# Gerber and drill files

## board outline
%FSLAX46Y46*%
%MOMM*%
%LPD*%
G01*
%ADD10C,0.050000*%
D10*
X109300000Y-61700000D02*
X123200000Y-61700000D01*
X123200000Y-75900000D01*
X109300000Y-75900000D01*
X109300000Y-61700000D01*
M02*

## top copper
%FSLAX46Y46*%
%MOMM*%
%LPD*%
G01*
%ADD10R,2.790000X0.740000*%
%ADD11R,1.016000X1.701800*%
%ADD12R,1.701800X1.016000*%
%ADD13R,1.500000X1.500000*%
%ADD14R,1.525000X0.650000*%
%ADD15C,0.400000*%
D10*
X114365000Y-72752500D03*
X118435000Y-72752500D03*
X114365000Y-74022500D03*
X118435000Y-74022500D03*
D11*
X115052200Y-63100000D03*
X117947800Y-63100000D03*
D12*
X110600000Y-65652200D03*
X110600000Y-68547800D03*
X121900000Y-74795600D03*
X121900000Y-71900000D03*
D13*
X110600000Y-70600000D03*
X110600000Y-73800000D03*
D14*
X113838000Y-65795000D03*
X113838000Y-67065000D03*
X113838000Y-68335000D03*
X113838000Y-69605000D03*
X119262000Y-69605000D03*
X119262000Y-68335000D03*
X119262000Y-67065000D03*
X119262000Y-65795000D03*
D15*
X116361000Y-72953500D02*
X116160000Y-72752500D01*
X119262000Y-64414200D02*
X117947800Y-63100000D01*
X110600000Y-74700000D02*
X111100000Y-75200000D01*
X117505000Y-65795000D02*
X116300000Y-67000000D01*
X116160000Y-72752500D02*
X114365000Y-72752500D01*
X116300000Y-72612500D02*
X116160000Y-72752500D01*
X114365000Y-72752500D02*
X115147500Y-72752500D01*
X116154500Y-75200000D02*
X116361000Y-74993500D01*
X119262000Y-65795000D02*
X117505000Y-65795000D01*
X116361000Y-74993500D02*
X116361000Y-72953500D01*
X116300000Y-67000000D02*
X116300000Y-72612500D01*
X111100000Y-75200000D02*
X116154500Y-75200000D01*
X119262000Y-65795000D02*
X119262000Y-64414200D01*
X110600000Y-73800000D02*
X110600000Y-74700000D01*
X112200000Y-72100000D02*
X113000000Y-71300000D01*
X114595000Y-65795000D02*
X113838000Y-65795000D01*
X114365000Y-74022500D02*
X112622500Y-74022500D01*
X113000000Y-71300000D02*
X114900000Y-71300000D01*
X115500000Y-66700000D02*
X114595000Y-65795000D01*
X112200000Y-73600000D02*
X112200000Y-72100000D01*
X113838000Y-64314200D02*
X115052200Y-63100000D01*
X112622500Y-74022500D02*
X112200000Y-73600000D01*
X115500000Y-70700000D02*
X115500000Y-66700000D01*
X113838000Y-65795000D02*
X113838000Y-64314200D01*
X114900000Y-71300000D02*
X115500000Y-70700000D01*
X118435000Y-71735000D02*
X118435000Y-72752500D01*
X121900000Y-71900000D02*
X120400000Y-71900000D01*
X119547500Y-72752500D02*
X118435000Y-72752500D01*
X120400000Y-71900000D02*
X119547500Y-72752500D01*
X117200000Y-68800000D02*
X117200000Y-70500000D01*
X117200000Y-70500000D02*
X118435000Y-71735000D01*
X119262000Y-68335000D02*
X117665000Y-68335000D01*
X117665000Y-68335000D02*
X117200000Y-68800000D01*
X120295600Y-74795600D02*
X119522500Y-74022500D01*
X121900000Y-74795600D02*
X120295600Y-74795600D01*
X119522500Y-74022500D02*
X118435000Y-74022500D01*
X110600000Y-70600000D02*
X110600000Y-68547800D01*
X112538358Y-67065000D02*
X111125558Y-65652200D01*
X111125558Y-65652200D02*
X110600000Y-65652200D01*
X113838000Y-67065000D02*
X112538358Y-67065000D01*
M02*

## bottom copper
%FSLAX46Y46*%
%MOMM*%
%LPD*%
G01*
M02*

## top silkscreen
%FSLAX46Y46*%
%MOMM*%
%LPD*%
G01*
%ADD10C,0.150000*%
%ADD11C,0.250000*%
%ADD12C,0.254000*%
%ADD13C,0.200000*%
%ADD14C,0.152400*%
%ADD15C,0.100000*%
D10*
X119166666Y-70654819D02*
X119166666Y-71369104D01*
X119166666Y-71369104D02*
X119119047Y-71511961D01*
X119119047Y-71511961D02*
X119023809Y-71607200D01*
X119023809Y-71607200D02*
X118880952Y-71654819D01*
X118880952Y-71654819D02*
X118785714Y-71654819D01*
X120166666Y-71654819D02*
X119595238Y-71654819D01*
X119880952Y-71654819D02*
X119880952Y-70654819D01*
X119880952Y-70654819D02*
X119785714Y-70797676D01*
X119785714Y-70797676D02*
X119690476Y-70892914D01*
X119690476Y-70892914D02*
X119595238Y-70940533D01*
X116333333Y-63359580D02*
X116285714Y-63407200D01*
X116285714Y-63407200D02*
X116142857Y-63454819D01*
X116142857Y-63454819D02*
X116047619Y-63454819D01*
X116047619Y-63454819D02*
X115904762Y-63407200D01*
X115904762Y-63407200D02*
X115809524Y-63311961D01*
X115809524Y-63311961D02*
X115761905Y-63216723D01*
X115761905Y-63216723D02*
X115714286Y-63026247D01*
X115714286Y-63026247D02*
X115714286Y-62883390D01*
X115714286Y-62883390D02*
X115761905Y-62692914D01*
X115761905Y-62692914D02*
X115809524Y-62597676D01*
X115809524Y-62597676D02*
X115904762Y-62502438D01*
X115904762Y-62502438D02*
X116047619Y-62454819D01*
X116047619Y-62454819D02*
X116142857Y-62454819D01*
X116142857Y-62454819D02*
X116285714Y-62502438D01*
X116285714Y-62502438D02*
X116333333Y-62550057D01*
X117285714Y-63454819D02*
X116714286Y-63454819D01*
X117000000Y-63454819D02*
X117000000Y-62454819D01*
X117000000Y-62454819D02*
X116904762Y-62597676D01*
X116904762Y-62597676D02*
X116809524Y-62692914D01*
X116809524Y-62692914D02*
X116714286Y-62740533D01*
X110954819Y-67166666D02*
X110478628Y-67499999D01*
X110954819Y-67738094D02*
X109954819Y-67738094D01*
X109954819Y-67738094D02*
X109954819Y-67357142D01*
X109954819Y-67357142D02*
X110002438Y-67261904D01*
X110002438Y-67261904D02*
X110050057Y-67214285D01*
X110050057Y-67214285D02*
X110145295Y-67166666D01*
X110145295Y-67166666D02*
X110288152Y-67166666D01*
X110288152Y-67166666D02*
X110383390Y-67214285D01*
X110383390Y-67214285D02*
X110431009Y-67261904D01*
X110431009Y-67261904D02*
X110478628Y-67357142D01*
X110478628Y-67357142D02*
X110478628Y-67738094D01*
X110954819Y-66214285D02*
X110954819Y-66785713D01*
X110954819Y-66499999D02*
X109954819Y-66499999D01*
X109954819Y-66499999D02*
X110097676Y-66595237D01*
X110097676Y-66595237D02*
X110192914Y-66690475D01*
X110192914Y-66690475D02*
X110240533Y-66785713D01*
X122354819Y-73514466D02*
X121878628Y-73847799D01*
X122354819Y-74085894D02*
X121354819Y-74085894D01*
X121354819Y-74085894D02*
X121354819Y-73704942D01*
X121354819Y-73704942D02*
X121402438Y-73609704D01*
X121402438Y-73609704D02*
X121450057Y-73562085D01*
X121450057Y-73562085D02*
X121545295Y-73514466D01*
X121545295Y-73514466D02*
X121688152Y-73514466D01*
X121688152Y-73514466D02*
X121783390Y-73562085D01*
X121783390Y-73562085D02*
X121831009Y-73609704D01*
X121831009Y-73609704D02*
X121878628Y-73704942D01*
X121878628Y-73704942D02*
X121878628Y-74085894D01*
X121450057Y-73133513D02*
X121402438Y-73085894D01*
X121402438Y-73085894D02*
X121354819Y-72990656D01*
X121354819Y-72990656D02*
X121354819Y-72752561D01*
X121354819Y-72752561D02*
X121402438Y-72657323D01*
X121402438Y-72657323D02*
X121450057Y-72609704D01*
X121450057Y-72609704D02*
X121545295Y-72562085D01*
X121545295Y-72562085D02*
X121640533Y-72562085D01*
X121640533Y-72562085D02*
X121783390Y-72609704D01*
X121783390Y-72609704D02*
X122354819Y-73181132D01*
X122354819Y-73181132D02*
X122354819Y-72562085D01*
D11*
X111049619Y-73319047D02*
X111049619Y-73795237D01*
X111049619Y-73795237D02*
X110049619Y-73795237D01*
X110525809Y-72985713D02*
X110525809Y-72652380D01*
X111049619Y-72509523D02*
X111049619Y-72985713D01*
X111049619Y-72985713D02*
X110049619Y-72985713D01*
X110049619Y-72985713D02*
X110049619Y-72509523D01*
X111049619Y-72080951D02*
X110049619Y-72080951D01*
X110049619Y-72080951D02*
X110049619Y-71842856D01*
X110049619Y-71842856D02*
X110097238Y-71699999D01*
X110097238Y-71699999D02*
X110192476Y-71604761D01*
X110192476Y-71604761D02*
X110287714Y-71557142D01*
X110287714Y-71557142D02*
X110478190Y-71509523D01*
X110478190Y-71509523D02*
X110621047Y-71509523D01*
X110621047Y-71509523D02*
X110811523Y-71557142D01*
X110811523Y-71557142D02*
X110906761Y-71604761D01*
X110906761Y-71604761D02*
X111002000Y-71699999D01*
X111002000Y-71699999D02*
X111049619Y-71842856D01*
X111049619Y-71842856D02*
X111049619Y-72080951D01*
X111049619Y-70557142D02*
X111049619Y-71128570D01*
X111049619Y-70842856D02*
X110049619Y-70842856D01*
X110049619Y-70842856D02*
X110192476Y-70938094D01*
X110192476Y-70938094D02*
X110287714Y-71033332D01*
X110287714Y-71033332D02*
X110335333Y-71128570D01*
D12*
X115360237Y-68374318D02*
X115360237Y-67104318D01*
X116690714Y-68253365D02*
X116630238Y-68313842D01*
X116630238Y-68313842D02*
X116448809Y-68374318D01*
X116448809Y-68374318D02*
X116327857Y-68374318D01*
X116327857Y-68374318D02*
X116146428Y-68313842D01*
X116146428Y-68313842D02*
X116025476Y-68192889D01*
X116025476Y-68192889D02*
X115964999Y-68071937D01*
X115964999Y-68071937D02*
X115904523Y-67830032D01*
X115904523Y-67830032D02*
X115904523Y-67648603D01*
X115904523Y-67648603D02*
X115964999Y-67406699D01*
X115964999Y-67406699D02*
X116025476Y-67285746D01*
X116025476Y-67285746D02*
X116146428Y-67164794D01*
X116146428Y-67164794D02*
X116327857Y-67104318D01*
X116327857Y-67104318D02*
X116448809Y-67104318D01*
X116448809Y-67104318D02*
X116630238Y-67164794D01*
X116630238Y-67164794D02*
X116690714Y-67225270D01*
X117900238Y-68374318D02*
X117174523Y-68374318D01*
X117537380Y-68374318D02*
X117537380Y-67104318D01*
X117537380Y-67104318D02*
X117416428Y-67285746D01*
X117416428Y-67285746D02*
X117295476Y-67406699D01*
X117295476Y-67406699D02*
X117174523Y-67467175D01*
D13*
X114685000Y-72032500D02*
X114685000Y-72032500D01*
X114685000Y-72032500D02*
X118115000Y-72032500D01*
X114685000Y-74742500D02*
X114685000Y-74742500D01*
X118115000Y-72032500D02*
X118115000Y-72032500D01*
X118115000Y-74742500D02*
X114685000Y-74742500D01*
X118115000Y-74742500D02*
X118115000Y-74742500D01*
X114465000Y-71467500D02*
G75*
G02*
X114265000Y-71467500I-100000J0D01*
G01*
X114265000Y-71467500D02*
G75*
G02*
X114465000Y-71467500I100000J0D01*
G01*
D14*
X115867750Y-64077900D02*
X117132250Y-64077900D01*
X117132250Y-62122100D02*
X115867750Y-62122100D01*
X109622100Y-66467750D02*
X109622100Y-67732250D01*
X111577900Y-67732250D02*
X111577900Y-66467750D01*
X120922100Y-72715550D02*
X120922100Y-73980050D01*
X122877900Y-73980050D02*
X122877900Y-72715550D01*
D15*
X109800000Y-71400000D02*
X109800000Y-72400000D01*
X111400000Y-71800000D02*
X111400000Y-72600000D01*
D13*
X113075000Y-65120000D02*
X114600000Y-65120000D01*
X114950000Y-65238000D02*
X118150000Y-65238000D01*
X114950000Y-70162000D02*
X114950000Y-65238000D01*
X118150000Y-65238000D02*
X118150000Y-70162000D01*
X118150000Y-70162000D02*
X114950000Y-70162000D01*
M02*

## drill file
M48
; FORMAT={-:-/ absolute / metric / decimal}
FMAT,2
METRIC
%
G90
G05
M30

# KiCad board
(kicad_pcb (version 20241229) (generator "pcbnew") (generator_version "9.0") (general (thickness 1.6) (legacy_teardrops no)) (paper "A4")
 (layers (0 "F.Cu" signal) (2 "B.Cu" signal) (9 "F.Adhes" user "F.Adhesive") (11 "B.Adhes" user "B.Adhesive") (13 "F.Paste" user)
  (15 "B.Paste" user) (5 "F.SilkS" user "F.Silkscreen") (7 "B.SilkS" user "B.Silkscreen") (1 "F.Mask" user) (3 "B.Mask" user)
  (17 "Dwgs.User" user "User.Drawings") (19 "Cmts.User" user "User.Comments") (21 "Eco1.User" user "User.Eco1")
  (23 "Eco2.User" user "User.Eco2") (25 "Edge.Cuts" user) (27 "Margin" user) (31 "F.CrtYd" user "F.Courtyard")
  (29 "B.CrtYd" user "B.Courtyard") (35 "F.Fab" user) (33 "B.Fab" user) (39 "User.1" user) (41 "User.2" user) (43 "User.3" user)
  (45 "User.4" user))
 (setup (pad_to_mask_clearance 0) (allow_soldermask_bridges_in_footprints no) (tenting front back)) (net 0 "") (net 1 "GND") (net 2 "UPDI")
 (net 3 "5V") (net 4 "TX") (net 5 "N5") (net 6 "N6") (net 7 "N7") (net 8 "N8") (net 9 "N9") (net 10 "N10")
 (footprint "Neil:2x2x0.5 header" (layer "F.Cu") (at 116.4 73.3875 -90)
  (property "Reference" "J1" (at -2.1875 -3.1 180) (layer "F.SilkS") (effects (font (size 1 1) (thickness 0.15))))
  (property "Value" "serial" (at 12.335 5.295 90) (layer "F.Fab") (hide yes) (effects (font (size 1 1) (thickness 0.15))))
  (fp_line (start -1.355 1.715) (end -1.355 1.715) (stroke (width 0.2) (type solid)) (layer "F.SilkS"))
  (fp_line (start -1.355 1.715) (end -1.355 -1.715) (stroke (width 0.2) (type solid)) (layer "F.SilkS"))
  (fp_line (start 1.355 1.715) (end 1.355 1.715) (stroke (width 0.2) (type solid)) (layer "F.SilkS"))
  (fp_line (start -1.355 -1.715) (end -1.355 -1.715) (stroke (width 0.2) (type solid)) (layer "F.SilkS"))
  (fp_line (start 1.355 -1.715) (end 1.355 1.715) (stroke (width 0.2) (type solid)) (layer "F.SilkS"))
  (fp_line (start 1.355 -1.715) (end 1.355 -1.715) (stroke (width 0.2) (type solid)) (layer "F.SilkS"))
  (fp_circle (center -1.92 2.035) (end -1.82 2.035) (stroke (width 0.2) (type solid)) (fill no) (layer "F.SilkS"))
  (pad "01" smd rect (at -0.635 2.035 270) (size 0.74 2.79) (layers "F.Cu" "F.Mask" "F.Paste") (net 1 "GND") (solder_mask_margin 0.102))
  (pad "02" smd rect (at -0.635 -2.035 270) (size 0.74 2.79) (layers "F.Cu" "F.Mask" "F.Paste") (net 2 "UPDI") (solder_mask_margin 0.102))
  (pad "03" smd rect (at 0.635 2.035 270) (size 0.74 2.79) (layers "F.Cu" "F.Mask" "F.Paste") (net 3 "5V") (solder_mask_margin 0.102))
  (pad "04" smd rect (at 0.635 -2.035 270) (size 0.74 2.79) (layers "F.Cu" "F.Mask" "F.Paste") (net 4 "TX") (solder_mask_margin 0.102)))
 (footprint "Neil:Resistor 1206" (layer "F.Cu") (at 116.5 63.1)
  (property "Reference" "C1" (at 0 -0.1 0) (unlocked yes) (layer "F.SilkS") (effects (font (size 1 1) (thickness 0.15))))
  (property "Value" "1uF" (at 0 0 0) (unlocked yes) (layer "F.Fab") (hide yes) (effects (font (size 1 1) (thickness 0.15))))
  (fp_line (start -0.63225 0.9779) (end 0.63225 0.9779) (stroke (width 0.1524) (type solid)) (layer "F.SilkS"))
  (fp_line (start 0.63225 -0.9779) (end -0.63225 -0.9779) (stroke (width 0.1524) (type solid)) (layer "F.SilkS"))
  (pad "1" smd rect (at -1.4478 0) (size 1.016 1.7018) (layers "F.Cu" "F.Mask" "F.Paste") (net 3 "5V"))
  (pad "2" smd rect (at 1.4478 0) (size 1.016 1.7018) (layers "F.Cu" "F.Mask" "F.Paste") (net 1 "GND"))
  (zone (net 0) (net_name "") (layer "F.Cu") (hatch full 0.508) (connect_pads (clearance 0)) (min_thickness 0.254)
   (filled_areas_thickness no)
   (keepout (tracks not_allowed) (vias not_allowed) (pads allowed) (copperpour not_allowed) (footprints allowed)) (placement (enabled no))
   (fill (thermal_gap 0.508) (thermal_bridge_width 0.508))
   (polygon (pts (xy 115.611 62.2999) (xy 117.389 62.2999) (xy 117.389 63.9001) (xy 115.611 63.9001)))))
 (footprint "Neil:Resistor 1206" (layer "F.Cu") (at 110.6 67.1 -90)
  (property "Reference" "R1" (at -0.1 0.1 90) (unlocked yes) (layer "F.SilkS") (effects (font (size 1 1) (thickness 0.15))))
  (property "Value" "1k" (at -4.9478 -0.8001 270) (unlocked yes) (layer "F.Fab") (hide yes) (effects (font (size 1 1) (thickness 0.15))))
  (fp_line (start -0.63225 0.9779) (end 0.63225 0.9779) (stroke (width 0.1524) (type solid)) (layer "F.SilkS"))
  (fp_line (start 0.63225 -0.9779) (end -0.63225 -0.9779) (stroke (width 0.1524) (type solid)) (layer "F.SilkS"))
  (pad "1" smd rect (at -1.4478 0 270) (size 1.016 1.7018) (layers "F.Cu" "F.Mask" "F.Paste") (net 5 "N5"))
  (pad "2" smd rect (at 1.4478 0 270) (size 1.016 1.7018) (layers "F.Cu" "F.Mask" "F.Paste") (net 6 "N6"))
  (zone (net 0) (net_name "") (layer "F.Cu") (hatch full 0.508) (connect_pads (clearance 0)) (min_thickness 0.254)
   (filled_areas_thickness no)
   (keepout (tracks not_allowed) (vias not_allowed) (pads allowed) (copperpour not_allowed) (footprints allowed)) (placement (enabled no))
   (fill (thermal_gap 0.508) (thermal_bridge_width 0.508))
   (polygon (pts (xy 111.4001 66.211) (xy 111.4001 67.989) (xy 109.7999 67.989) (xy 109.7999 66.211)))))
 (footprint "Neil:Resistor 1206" (layer "F.Cu") (at 121.9 73.3478 90)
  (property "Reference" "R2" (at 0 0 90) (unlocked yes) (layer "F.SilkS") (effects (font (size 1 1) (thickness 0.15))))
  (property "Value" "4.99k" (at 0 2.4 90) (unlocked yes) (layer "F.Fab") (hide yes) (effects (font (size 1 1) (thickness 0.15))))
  (fp_line (start 0.63225 -0.9779) (end -0.63225 -0.9779) (stroke (width 0.1524) (type solid)) (layer "F.SilkS"))
  (fp_line (start -0.63225 0.9779) (end 0.63225 0.9779) (stroke (width 0.1524) (type solid)) (layer "F.SilkS"))
  (pad "1" smd rect (at -1.4478 0 90) (size 1.016 1.7018) (layers "F.Cu" "F.Mask" "F.Paste") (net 4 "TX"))
  (pad "2" smd rect (at 1.4478 0 90) (size 1.016 1.7018) (layers "F.Cu" "F.Mask" "F.Paste") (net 2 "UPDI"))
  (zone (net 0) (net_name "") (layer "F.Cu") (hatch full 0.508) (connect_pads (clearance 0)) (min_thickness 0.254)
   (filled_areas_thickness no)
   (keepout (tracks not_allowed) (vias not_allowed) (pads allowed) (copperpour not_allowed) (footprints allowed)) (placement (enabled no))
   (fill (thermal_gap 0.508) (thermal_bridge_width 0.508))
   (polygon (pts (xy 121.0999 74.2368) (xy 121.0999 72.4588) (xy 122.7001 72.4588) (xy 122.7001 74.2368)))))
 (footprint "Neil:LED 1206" (layer "F.Cu") (at 110.6 72.2 -90)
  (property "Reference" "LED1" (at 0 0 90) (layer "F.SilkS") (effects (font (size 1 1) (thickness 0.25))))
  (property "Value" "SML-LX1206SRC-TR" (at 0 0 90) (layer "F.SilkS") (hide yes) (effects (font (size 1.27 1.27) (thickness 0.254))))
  (fp_line (start -0.8 0.8) (end 0.2 0.8) (stroke (width 0.1) (type solid)) (layer "F.SilkS"))
  (fp_line (start -0.4 -0.8) (end 0.4 -0.8) (stroke (width 0.1) (type solid)) (layer "F.SilkS"))
  (pad "1" smd rect (at -1.6 0) (size 1.5 1.5) (layers "F.Cu" "F.Mask" "F.Paste") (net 6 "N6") (thermal_bridge_angle 45))
  (pad "2" smd rect (at 1.6 0) (size 1.5 1.5) (layers "F.Cu" "F.Mask" "F.Paste") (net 1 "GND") (thermal_bridge_angle 45)))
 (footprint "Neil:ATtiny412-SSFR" (layer "F.Cu") (at 116.55 67.7)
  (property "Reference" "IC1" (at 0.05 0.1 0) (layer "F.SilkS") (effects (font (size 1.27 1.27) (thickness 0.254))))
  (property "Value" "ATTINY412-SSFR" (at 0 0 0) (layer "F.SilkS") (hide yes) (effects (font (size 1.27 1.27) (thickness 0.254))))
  (fp_line (start -3.475 -2.58) (end -1.95 -2.58) (stroke (width 0.2) (type solid)) (layer "F.SilkS"))
  (fp_line (start -1.6 -2.462) (end 1.6 -2.462) (stroke (width 0.2) (type solid)) (layer "F.SilkS"))
  (fp_line (start -1.6 2.462) (end -1.6 -2.462) (stroke (width 0.2) (type solid)) (layer "F.SilkS"))
  (fp_line (start 1.6 -2.462) (end 1.6 2.462) (stroke (width 0.2) (type solid)) (layer "F.SilkS"))
  (fp_line (start 1.6 2.462) (end -1.6 2.462) (stroke (width 0.2) (type solid)) (layer "F.SilkS"))
  (pad "1" smd rect (at -2.712 -1.905 90) (size 0.65 1.525) (layers "F.Cu" "F.Mask" "F.Paste") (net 3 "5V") (thermal_bridge_angle 45))
  (pad "2" smd rect (at -2.712 -0.635 90) (size 0.65 1.525) (layers "F.Cu" "F.Mask" "F.Paste") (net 5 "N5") (thermal_bridge_angle 45))
  (pad "3" smd rect (at -2.712 0.635 90) (size 0.65 1.525) (layers "F.Cu" "F.Mask" "F.Paste") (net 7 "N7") (thermal_bridge_angle 45))
  (pad "4" smd rect (at -2.712 1.905 90) (size 0.65 1.525) (layers "F.Cu" "F.Mask" "F.Paste") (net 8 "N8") (thermal_bridge_angle 45))
  (pad "5" smd rect (at 2.712 1.905 90) (size 0.65 1.525) (layers "F.Cu" "F.Mask" "F.Paste") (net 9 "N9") (thermal_bridge_angle 45))
  (pad "6" smd rect (at 2.712 0.635 90) (size 0.65 1.525) (layers "F.Cu" "F.Mask" "F.Paste") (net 2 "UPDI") (thermal_bridge_angle 45))
  (pad "7" smd rect (at 2.712 -0.635 90) (size 0.65 1.525) (layers "F.Cu" "F.Mask" "F.Paste") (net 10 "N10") (thermal_bridge_angle 45))
  (pad "8" smd rect (at 2.712 -1.905 90) (size 0.65 1.525) (layers "F.Cu" "F.Mask" "F.Paste") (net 1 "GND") (thermal_bridge_angle 45)))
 (gr_rect (start 109.3 61.7) (end 123.2 75.9) (stroke (width 0.05) (type default)) (fill no) (layer "Edge.Cuts"))
 (segment (start 116.361 72.9535) (end 116.16 72.7525) (width 0.4) (layer "F.Cu") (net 1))
 (segment (start 119.262 64.4142) (end 117.9478 63.1) (width 0.4) (layer "F.Cu") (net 1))
 (segment (start 110.6 74.7) (end 111.1 75.2) (width 0.4) (layer "F.Cu") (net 1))
 (segment (start 117.505 65.795) (end 116.3 67) (width 0.4) (layer "F.Cu") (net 1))
 (segment (start 116.16 72.7525) (end 114.365 72.7525) (width 0.4) (layer "F.Cu") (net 1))
 (segment (start 116.3 72.6125) (end 116.16 72.7525) (width 0.4) (layer "F.Cu") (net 1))
 (segment (start 114.365 72.7525) (end 115.1475 72.7525) (width 0.4) (layer "F.Cu") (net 1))
 (segment (start 116.1545 75.2) (end 116.361 74.9935) (width 0.4) (layer "F.Cu") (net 1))
 (segment (start 119.262 65.795) (end 117.505 65.795) (width 0.4) (layer "F.Cu") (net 1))
 (segment (start 116.361 74.9935) (end 116.361 72.9535) (width 0.4) (layer "F.Cu") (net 1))
 (segment (start 116.3 67) (end 116.3 72.6125) (width 0.4) (layer "F.Cu") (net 1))
 (segment (start 111.1 75.2) (end 116.1545 75.2) (width 0.4) (layer "F.Cu") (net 1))
 (segment (start 119.262 65.795) (end 119.262 64.4142) (width 0.4) (layer "F.Cu") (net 1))
 (segment (start 110.6 73.8) (end 110.6 74.7) (width 0.4) (layer "F.Cu") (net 1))
 (segment (start 112.2 72.1) (end 113 71.3) (width 0.4) (layer "F.Cu") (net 3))
 (segment (start 114.595 65.795) (end 113.838 65.795) (width 0.4) (layer "F.Cu") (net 3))
 (segment (start 114.365 74.0225) (end 112.6225 74.0225) (width 0.4) (layer "F.Cu") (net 3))
 (segment (start 113 71.3) (end 114.9 71.3) (width 0.4) (layer "F.Cu") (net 3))
 (segment (start 115.5 66.7) (end 114.595 65.795) (width 0.4) (layer "F.Cu") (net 3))
 (segment (start 112.2 73.6) (end 112.2 72.1) (width 0.4) (layer "F.Cu") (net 3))
 (segment (start 113.838 64.3142) (end 115.0522 63.1) (width 0.4) (layer "F.Cu") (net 3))
 (segment (start 112.6225 74.0225) (end 112.2 73.6) (width 0.4) (layer "F.Cu") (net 3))
 (segment (start 115.5 70.7) (end 115.5 66.7) (width 0.4) (layer "F.Cu") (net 3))
 (segment (start 113.838 65.795) (end 113.838 64.3142) (width 0.4) (layer "F.Cu") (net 3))
 (segment (start 114.9 71.3) (end 115.5 70.7) (width 0.4) (layer "F.Cu") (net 3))
 (segment (start 118.435 71.735) (end 118.435 72.7525) (width 0.4) (layer "F.Cu") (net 2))
 (segment (start 121.9 71.9) (end 120.4 71.9) (width 0.4) (layer "F.Cu") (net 2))
 (segment (start 119.5475 72.7525) (end 118.435 72.7525) (width 0.4) (layer "F.Cu") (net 2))
 (segment (start 120.4 71.9) (end 119.5475 72.7525) (width 0.4) (layer "F.Cu") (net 2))
 (segment (start 117.2 68.8) (end 117.2 70.5) (width 0.4) (layer "F.Cu") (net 2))
 (segment (start 117.2 70.5) (end 118.435 71.735) (width 0.4) (layer "F.Cu") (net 2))
 (segment (start 119.262 68.335) (end 117.665 68.335) (width 0.4) (layer "F.Cu") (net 2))
 (segment (start 117.665 68.335) (end 117.2 68.8) (width 0.4) (layer "F.Cu") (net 2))
 (segment (start 120.2956 74.7956) (end 119.5225 74.0225) (width 0.4) (layer "F.Cu") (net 4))
 (segment (start 121.9 74.7956) (end 120.2956 74.7956) (width 0.4) (layer "F.Cu") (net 4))
 (segment (start 119.5225 74.0225) (end 118.435 74.0225) (width 0.4) (layer "F.Cu") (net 4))
 (segment (start 110.6 70.6) (end 110.6 68.5478) (width 0.4) (layer "F.Cu") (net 6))
 (segment (start 112.538358 67.065) (end 111.125558 65.6522) (width 0.4) (layer "F.Cu") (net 5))
 (segment (start 111.125558 65.6522) (end 110.6 65.6522) (width 0.4) (layer "F.Cu") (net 5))
 (segment (start 113.838 67.065) (end 112.538358 67.065) (width 0.4) (layer "F.Cu") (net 5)))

